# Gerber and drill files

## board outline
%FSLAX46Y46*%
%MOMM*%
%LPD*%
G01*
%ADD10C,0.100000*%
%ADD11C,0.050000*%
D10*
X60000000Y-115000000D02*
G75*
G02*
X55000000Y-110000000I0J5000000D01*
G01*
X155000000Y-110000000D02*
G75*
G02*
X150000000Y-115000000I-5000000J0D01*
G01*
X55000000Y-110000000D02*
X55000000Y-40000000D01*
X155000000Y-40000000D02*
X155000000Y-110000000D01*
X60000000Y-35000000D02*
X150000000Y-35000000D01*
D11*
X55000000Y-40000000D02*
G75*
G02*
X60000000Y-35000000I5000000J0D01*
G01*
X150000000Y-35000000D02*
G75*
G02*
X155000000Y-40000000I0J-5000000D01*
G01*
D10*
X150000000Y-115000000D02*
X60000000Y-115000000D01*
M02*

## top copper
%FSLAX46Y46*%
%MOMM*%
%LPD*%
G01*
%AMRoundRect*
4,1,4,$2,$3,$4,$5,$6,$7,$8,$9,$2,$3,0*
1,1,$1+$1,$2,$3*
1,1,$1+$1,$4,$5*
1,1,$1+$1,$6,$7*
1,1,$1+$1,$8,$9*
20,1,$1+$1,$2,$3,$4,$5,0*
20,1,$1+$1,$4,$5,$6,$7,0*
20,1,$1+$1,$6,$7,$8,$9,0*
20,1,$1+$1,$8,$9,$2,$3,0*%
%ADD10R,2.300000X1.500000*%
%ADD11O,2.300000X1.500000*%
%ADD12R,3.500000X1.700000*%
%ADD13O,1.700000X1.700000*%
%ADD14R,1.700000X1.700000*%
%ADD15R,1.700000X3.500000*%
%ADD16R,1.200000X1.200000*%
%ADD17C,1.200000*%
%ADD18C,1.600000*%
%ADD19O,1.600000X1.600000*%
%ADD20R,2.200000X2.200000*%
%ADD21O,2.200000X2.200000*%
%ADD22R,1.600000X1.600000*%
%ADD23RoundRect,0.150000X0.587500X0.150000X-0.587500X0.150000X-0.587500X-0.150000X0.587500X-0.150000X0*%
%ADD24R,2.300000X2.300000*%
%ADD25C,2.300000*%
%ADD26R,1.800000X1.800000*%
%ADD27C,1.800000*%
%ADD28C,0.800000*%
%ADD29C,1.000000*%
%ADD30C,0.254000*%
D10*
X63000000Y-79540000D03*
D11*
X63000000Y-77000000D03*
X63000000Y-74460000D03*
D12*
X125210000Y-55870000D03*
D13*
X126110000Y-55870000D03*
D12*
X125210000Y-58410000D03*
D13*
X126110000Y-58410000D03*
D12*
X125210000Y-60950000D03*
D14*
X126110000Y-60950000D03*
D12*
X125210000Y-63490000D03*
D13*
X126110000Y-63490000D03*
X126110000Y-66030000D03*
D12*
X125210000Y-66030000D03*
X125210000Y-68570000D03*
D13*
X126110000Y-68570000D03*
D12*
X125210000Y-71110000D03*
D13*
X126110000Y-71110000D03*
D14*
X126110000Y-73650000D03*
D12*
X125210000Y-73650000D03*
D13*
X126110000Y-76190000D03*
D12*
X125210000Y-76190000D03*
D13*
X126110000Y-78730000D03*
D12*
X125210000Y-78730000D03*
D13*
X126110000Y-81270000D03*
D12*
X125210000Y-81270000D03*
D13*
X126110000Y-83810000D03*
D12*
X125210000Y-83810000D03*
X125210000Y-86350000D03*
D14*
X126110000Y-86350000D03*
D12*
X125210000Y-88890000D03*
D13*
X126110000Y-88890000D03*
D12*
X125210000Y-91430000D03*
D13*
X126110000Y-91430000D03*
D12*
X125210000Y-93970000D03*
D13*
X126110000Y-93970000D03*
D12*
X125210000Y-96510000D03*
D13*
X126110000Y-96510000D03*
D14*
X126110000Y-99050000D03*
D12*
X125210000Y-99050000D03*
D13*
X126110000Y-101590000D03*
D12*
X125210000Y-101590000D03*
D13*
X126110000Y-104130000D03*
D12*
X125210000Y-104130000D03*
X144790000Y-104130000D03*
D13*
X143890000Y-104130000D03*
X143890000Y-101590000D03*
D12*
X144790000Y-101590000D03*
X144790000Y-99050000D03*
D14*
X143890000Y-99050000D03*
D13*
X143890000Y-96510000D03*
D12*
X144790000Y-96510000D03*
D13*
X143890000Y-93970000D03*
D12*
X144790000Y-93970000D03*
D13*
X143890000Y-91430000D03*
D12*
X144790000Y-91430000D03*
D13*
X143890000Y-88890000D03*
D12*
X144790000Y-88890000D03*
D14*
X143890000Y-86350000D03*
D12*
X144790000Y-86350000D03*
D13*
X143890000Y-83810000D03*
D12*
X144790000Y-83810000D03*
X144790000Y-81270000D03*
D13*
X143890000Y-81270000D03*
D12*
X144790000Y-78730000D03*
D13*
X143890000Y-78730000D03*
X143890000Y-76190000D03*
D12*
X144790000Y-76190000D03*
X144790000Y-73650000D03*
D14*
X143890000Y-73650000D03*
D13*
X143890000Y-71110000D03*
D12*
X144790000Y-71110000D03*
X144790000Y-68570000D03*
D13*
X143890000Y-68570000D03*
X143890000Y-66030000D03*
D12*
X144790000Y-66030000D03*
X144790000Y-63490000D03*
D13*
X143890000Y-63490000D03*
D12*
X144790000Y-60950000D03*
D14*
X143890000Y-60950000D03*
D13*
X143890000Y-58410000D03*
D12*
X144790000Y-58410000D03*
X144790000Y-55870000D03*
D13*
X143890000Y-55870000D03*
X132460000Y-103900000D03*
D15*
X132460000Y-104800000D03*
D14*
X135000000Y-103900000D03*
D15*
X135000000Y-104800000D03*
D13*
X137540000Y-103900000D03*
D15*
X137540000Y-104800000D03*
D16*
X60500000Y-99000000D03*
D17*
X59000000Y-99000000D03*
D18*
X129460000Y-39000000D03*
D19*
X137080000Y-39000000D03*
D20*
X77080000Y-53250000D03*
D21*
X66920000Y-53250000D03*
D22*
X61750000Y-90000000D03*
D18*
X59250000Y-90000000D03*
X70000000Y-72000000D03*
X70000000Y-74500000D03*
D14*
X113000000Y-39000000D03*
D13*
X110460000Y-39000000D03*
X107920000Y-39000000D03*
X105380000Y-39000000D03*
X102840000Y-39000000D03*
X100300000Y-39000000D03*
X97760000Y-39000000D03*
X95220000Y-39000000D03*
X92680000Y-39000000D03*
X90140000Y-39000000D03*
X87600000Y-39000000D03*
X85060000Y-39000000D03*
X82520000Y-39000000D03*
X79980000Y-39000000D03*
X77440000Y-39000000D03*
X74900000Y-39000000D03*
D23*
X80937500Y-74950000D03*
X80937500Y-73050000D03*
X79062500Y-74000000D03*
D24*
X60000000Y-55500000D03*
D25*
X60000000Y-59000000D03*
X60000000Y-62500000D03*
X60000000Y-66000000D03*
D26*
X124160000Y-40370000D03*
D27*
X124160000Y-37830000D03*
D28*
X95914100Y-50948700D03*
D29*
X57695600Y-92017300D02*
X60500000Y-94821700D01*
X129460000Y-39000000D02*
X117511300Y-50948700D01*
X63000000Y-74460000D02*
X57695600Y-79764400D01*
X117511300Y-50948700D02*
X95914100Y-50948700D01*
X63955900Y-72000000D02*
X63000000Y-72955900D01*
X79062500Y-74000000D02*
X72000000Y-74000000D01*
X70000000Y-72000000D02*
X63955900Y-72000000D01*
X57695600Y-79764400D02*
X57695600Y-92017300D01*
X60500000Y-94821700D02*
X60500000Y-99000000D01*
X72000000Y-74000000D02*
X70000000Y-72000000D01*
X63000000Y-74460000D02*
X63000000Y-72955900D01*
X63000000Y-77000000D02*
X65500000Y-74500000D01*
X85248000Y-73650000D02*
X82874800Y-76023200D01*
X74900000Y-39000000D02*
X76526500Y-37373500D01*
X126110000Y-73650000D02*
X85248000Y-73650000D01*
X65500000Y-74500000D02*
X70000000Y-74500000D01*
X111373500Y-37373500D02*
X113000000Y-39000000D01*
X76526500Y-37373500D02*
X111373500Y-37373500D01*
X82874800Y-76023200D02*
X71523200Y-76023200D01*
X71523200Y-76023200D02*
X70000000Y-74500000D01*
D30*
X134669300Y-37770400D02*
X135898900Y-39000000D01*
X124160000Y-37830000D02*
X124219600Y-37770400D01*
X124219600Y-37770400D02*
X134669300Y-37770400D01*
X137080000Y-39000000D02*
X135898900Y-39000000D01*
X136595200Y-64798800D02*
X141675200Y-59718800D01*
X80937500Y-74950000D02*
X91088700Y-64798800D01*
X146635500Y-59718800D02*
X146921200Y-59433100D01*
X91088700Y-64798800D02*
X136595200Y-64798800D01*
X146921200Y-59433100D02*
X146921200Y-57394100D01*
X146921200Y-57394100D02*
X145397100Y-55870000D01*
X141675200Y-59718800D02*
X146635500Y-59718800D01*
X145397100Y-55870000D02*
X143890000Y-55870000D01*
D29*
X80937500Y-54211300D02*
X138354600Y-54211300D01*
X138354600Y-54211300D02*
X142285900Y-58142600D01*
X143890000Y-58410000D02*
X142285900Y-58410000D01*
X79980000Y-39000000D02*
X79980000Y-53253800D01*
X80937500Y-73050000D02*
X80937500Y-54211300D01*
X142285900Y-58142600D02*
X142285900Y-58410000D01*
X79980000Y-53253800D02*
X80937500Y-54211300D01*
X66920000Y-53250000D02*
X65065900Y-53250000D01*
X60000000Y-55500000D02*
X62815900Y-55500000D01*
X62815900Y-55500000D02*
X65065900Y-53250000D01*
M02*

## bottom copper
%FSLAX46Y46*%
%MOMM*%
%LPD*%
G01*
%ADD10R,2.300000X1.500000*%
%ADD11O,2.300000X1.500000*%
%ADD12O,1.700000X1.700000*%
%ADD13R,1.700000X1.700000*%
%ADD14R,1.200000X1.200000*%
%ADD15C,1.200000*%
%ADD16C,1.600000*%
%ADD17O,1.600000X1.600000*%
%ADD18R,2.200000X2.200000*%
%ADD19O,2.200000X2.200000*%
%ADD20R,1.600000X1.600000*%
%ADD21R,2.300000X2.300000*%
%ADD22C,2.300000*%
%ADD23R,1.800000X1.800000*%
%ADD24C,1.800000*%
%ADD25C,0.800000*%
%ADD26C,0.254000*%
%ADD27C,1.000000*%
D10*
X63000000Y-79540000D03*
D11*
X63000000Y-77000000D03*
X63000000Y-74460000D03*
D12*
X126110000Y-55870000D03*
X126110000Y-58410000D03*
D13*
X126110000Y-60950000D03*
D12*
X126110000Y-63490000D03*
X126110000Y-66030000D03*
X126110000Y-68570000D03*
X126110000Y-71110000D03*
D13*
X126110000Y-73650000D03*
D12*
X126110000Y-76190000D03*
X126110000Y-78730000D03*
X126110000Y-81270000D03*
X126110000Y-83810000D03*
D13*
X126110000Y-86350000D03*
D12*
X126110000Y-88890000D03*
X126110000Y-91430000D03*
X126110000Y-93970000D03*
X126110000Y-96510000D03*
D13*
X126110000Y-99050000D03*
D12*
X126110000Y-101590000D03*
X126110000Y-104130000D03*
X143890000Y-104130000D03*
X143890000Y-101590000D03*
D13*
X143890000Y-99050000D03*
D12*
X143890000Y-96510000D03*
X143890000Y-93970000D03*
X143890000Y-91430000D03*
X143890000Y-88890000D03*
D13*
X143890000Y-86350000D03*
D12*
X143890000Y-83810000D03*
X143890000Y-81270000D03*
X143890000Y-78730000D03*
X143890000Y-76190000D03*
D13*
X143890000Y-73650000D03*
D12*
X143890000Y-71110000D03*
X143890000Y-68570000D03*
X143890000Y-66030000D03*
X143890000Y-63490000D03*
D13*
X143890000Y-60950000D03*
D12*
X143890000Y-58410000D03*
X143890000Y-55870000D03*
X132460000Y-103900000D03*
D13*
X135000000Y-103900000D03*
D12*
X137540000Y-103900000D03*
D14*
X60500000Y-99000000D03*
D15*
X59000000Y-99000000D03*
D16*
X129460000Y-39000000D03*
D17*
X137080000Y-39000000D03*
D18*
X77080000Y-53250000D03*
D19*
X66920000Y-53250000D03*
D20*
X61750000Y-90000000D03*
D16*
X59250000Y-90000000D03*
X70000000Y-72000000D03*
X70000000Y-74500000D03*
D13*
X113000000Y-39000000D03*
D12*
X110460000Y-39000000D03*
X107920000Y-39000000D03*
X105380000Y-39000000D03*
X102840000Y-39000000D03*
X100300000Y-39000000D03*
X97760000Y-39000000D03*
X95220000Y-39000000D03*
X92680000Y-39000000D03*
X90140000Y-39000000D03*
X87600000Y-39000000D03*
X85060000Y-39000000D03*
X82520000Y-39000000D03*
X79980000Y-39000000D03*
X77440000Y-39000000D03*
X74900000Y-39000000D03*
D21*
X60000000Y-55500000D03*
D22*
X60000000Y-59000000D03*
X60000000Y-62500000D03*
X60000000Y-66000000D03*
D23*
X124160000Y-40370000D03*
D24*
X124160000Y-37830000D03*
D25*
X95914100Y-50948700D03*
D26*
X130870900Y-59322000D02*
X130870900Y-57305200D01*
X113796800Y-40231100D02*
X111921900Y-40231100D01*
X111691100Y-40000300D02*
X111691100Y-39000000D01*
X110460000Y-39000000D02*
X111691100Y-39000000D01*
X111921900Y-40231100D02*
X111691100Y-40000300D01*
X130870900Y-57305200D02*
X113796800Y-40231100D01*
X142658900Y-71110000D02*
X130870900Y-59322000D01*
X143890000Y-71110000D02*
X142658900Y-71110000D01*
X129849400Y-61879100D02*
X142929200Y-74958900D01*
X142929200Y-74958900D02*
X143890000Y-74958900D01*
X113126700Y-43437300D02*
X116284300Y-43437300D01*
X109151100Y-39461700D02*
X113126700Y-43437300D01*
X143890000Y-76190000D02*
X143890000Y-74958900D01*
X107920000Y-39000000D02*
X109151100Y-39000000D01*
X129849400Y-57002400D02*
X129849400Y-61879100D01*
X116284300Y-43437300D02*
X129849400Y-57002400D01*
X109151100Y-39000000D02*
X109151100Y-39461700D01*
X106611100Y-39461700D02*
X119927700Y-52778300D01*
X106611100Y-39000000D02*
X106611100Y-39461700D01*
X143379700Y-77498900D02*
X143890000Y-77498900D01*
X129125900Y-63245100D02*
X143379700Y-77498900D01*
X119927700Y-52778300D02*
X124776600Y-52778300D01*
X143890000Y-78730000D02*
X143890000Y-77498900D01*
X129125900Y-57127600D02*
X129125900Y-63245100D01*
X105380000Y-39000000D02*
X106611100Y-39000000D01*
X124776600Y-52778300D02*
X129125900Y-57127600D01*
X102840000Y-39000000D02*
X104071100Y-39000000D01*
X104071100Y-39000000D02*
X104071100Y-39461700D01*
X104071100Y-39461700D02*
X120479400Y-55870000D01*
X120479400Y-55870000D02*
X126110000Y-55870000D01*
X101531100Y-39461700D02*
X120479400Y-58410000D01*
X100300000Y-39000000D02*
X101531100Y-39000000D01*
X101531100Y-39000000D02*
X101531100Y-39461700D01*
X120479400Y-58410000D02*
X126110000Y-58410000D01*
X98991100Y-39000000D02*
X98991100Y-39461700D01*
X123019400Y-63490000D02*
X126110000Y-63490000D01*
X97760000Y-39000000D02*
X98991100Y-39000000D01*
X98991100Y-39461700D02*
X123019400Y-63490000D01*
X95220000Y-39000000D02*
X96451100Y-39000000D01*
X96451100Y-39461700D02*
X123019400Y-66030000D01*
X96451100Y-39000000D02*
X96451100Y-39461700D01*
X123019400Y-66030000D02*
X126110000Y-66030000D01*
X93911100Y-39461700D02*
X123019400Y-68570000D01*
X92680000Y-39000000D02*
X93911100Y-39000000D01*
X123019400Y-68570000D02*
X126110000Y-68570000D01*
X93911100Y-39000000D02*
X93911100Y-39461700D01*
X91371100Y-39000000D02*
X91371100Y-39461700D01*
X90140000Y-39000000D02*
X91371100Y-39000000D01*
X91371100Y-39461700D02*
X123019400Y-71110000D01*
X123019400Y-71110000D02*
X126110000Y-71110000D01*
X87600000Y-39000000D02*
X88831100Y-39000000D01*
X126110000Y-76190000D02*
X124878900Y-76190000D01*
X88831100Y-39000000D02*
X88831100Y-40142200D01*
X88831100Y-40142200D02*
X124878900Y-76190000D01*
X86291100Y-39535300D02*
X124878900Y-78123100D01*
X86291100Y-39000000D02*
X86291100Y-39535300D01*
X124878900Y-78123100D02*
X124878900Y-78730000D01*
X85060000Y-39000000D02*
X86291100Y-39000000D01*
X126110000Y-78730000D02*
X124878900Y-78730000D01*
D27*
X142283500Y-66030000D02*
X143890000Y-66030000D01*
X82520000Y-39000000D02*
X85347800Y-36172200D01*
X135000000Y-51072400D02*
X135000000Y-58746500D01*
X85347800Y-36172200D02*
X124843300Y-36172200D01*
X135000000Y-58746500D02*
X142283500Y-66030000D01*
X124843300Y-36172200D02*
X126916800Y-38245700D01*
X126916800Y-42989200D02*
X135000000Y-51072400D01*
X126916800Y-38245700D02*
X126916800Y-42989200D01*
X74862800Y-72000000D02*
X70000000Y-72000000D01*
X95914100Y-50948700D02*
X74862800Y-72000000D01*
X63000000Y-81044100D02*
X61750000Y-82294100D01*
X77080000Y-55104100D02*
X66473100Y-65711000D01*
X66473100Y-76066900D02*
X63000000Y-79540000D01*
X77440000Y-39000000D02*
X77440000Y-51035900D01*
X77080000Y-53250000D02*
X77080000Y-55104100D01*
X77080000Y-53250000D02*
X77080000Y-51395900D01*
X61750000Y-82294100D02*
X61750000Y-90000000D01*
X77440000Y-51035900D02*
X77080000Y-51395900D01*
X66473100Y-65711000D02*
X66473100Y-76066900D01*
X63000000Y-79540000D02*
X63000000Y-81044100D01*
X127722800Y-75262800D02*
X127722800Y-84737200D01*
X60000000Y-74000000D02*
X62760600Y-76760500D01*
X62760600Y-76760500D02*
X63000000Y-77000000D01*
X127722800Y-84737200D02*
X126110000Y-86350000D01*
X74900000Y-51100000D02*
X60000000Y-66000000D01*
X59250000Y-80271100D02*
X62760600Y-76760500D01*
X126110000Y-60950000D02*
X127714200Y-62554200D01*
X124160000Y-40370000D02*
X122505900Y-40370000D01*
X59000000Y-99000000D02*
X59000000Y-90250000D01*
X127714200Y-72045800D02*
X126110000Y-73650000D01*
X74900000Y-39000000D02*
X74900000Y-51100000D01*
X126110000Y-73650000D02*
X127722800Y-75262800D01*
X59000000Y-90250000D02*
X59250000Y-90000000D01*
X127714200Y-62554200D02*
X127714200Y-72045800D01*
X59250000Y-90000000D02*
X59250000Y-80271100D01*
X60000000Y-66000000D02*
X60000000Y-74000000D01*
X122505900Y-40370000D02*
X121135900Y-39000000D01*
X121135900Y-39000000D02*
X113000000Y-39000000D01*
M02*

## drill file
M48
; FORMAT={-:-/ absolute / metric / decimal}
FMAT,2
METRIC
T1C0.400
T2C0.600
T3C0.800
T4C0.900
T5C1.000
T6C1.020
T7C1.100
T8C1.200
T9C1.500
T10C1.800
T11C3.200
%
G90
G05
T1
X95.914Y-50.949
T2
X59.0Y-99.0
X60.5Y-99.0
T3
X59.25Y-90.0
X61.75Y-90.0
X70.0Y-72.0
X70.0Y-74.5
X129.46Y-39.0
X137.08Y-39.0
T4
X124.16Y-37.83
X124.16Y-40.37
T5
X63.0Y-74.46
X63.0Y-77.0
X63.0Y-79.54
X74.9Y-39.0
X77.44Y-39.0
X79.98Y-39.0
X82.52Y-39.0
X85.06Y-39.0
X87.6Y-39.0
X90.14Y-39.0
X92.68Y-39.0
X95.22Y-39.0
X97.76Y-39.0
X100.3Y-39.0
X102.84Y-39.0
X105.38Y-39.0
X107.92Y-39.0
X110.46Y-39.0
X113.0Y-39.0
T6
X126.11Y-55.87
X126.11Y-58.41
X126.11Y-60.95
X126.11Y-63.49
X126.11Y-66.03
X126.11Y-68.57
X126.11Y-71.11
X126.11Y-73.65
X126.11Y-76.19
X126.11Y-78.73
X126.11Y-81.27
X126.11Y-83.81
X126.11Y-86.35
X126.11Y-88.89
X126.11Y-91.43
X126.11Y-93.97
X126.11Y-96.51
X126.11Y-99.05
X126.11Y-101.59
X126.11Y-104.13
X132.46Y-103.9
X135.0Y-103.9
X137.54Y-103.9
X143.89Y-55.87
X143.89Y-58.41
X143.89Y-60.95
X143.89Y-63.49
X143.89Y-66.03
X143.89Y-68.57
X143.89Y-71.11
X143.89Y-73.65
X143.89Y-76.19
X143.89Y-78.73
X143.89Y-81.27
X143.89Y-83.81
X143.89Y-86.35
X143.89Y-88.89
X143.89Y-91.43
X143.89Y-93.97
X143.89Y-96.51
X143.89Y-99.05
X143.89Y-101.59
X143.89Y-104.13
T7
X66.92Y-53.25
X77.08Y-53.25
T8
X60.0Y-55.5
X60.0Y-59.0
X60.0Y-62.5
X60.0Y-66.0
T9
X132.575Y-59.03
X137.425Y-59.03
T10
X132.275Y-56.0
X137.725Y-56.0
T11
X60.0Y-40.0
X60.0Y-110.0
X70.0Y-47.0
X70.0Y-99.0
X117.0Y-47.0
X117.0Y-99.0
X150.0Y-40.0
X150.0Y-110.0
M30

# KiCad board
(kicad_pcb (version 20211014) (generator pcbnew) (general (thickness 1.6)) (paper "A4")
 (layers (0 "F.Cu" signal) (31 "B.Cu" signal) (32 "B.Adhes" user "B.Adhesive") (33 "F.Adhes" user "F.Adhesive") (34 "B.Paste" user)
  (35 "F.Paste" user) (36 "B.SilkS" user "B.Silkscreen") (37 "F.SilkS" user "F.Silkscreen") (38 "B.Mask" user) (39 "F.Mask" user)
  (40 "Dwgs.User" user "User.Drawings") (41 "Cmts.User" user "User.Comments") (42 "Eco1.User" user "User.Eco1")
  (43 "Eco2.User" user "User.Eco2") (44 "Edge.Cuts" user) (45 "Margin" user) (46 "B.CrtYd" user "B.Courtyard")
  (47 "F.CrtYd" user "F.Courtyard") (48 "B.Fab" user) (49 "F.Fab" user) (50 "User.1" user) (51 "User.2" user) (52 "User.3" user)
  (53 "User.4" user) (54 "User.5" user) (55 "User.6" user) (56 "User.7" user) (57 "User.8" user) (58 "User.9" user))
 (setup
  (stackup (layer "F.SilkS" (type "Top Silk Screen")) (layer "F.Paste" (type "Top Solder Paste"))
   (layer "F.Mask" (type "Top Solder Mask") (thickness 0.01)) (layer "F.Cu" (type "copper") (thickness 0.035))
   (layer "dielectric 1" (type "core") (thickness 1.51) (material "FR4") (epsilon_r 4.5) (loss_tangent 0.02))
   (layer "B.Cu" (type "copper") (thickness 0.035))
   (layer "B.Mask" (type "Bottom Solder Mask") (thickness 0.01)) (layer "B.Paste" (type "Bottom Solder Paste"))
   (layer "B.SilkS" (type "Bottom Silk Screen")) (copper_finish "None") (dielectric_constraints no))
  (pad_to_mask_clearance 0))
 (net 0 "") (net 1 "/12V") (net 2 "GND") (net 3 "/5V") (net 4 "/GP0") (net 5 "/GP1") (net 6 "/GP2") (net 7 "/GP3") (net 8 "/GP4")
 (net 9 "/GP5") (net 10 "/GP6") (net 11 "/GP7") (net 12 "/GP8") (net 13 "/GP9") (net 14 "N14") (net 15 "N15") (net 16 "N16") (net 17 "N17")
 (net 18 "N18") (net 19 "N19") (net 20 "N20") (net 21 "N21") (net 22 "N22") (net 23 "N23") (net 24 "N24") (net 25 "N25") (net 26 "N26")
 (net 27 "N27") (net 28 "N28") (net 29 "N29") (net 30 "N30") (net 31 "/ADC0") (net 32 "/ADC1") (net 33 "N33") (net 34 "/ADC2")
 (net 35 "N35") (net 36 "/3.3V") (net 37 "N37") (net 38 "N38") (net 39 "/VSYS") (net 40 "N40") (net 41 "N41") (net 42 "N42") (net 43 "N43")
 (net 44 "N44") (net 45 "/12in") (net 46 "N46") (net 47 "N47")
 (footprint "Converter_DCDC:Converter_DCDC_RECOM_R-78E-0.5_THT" (layer "F.Cu") (at 63 79.54 90)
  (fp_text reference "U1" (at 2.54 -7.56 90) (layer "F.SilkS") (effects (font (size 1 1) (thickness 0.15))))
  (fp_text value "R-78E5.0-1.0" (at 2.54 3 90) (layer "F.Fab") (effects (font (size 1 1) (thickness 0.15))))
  (pad "1" thru_hole rect (at 0 0 90) (size 1.5 2.3) (drill 1) (layers *.Cu *.Mask) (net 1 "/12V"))
  (pad "2" thru_hole oval (at 2.54 0 90) (size 1.5 2.3) (drill 1) (layers *.Cu *.Mask) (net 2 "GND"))
  (pad "3" thru_hole oval (at 5.08 0 90) (size 1.5 2.3) (drill 1) (layers *.Cu *.Mask) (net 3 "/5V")))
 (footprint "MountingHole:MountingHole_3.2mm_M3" (layer "F.Cu") (at 117 99)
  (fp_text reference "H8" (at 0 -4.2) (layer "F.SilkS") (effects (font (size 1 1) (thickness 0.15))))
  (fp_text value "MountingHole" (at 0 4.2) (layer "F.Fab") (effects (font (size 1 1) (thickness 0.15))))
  (pad "" np_thru_hole circle (at 0 0) (size 3.2 3.2) (drill 3.2) (layers *.Cu *.Mask)))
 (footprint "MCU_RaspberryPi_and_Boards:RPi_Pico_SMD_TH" (layer "F.Cu") (at 135 80)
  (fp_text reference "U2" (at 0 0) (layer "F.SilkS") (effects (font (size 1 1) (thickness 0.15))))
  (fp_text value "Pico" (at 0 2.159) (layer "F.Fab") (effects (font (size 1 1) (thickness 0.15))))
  (pad "" np_thru_hole oval (at -2.725 -24) (size 1.8 1.8) (drill 1.8) (layers *.Cu *.Mask))
  (pad "" np_thru_hole oval (at -2.425 -20.97) (size 1.5 1.5) (drill 1.5) (layers *.Cu *.Mask))
  (pad "" np_thru_hole oval (at 2.425 -20.97) (size 1.5 1.5) (drill 1.5) (layers *.Cu *.Mask))
  (pad "" np_thru_hole oval (at 2.725 -24) (size 1.8 1.8) (drill 1.8) (layers *.Cu *.Mask))
  (pad "1" smd rect (at -8.89 -24.13) (size 3.5 1.7) (drill (offset -0.9 0)) (layers "F.Cu" "F.Mask") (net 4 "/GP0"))
  (pad "1" thru_hole oval (at -8.89 -24.13) (size 1.7 1.7) (drill 1.02) (layers *.Cu *.Mask) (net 4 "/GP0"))
  (pad "2" smd rect (at -8.89 -21.59) (size 3.5 1.7) (drill (offset -0.9 0)) (layers "F.Cu" "F.Mask") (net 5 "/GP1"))
  (pad "2" thru_hole oval (at -8.89 -21.59) (size 1.7 1.7) (drill 1.02) (layers *.Cu *.Mask) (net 5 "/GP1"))
  (pad "3" smd rect (at -8.89 -19.05) (size 3.5 1.7) (drill (offset -0.9 0)) (layers "F.Cu" "F.Mask") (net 2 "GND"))
  (pad "3" thru_hole rect (at -8.89 -19.05) (size 1.7 1.7) (drill 1.02) (layers *.Cu *.Mask) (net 2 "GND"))
  (pad "4" smd rect (at -8.89 -16.51) (size 3.5 1.7) (drill (offset -0.9 0)) (layers "F.Cu" "F.Mask") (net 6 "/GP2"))
  (pad "4" thru_hole oval (at -8.89 -16.51) (size 1.7 1.7) (drill 1.02) (layers *.Cu *.Mask) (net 6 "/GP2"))
  (pad "5" thru_hole oval (at -8.89 -13.97) (size 1.7 1.7) (drill 1.02) (layers *.Cu *.Mask) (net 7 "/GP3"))
  (pad "5" smd rect (at -8.89 -13.97) (size 3.5 1.7) (drill (offset -0.9 0)) (layers "F.Cu" "F.Mask") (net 7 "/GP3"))
  (pad "6" smd rect (at -8.89 -11.43) (size 3.5 1.7) (drill (offset -0.9 0)) (layers "F.Cu" "F.Mask") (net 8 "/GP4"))
  (pad "6" thru_hole oval (at -8.89 -11.43) (size 1.7 1.7) (drill 1.02) (layers *.Cu *.Mask) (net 8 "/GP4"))
  (pad "7" smd rect (at -8.89 -8.89) (size 3.5 1.7) (drill (offset -0.9 0)) (layers "F.Cu" "F.Mask") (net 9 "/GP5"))
  (pad "7" thru_hole oval (at -8.89 -8.89) (size 1.7 1.7) (drill 1.02) (layers *.Cu *.Mask) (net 9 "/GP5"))
  (pad "8" thru_hole rect (at -8.89 -6.35) (size 1.7 1.7) (drill 1.02) (layers *.Cu *.Mask) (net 2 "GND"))
  (pad "8" smd rect (at -8.89 -6.35) (size 3.5 1.7) (drill (offset -0.9 0)) (layers "F.Cu" "F.Mask") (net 2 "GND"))
  (pad "9" thru_hole oval (at -8.89 -3.81) (size 1.7 1.7) (drill 1.02) (layers *.Cu *.Mask) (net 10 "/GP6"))
  (pad "9" smd rect (at -8.89 -3.81) (size 3.5 1.7) (drill (offset -0.9 0)) (layers "F.Cu" "F.Mask") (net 10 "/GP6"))
  (pad "10" thru_hole oval (at -8.89 -1.27) (size 1.7 1.7) (drill 1.02) (layers *.Cu *.Mask) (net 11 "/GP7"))
  (pad "10" smd rect (at -8.89 -1.27) (size 3.5 1.7) (drill (offset -0.9 0)) (layers "F.Cu" "F.Mask") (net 11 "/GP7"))
  (pad "11" thru_hole oval (at -8.89 1.27) (size 1.7 1.7) (drill 1.02) (layers *.Cu *.Mask) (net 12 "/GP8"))
  (pad "11" smd rect (at -8.89 1.27) (size 3.5 1.7) (drill (offset -0.9 0)) (layers "F.Cu" "F.Mask") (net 12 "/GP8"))
  (pad "12" thru_hole oval (at -8.89 3.81) (size 1.7 1.7) (drill 1.02) (layers *.Cu *.Mask) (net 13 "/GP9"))
  (pad "12" smd rect (at -8.89 3.81) (size 3.5 1.7) (drill (offset -0.9 0)) (layers "F.Cu" "F.Mask") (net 13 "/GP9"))
  (pad "13" smd rect (at -8.89 6.35) (size 3.5 1.7) (drill (offset -0.9 0)) (layers "F.Cu" "F.Mask") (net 2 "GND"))
  (pad "13" thru_hole rect (at -8.89 6.35) (size 1.7 1.7) (drill 1.02) (layers *.Cu *.Mask) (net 2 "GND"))
  (pad "14" smd rect (at -8.89 8.89) (size 3.5 1.7) (drill (offset -0.9 0)) (layers "F.Cu" "F.Mask") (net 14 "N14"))
  (pad "14" thru_hole oval (at -8.89 8.89) (size 1.7 1.7) (drill 1.02) (layers *.Cu *.Mask) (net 14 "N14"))
  (pad "15" smd rect (at -8.89 11.43) (size 3.5 1.7) (drill (offset -0.9 0)) (layers "F.Cu" "F.Mask") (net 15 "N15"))
  (pad "15" thru_hole oval (at -8.89 11.43) (size 1.7 1.7) (drill 1.02) (layers *.Cu *.Mask) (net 15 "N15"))
  (pad "16" smd rect (at -8.89 13.97) (size 3.5 1.7) (drill (offset -0.9 0)) (layers "F.Cu" "F.Mask") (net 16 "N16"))
  (pad "16" thru_hole oval (at -8.89 13.97) (size 1.7 1.7) (drill 1.02) (layers *.Cu *.Mask) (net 16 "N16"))
  (pad "17" smd rect (at -8.89 16.51) (size 3.5 1.7) (drill (offset -0.9 0)) (layers "F.Cu" "F.Mask") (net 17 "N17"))
  (pad "17" thru_hole oval (at -8.89 16.51) (size 1.7 1.7) (drill 1.02) (layers *.Cu *.Mask) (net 17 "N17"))
  (pad "18" thru_hole rect (at -8.89 19.05) (size 1.7 1.7) (drill 1.02) (layers *.Cu *.Mask) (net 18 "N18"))
  (pad "18" smd rect (at -8.89 19.05) (size 3.5 1.7) (drill (offset -0.9 0)) (layers "F.Cu" "F.Mask") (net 18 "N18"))
  (pad "19" thru_hole oval (at -8.89 21.59) (size 1.7 1.7) (drill 1.02) (layers *.Cu *.Mask) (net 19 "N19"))
  (pad "19" smd rect (at -8.89 21.59) (size 3.5 1.7) (drill (offset -0.9 0)) (layers "F.Cu" "F.Mask") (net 19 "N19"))
  (pad "20" thru_hole oval (at -8.89 24.13) (size 1.7 1.7) (drill 1.02) (layers *.Cu *.Mask) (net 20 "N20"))
  (pad "20" smd rect (at -8.89 24.13) (size 3.5 1.7) (drill (offset -0.9 0)) (layers "F.Cu" "F.Mask") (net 20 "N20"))
  (pad "21" smd rect (at 8.89 24.13) (size 3.5 1.7) (drill (offset 0.9 0)) (layers "F.Cu" "F.Mask") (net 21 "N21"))
  (pad "21" thru_hole oval (at 8.89 24.13) (size 1.7 1.7) (drill 1.02) (layers *.Cu *.Mask) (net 21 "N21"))
  (pad "22" thru_hole oval (at 8.89 21.59) (size 1.7 1.7) (drill 1.02) (layers *.Cu *.Mask) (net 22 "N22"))
  (pad "22" smd rect (at 8.89 21.59) (size 3.5 1.7) (drill (offset 0.9 0)) (layers "F.Cu" "F.Mask") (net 22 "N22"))
  (pad "23" smd rect (at 8.89 19.05) (size 3.5 1.7) (drill (offset 0.9 0)) (layers "F.Cu" "F.Mask") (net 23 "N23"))
  (pad "23" thru_hole rect (at 8.89 19.05) (size 1.7 1.7) (drill 1.02) (layers *.Cu *.Mask) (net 23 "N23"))
  (pad "24" thru_hole oval (at 8.89 16.51) (size 1.7 1.7) (drill 1.02) (layers *.Cu *.Mask) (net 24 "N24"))
  (pad "24" smd rect (at 8.89 16.51) (size 3.5 1.7) (drill (offset 0.9 0)) (layers "F.Cu" "F.Mask") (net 24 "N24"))
  (pad "25" thru_hole oval (at 8.89 13.97) (size 1.7 1.7) (drill 1.02) (layers *.Cu *.Mask) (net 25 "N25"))
  (pad "25" smd rect (at 8.89 13.97) (size 3.5 1.7) (drill (offset 0.9 0)) (layers "F.Cu" "F.Mask") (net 25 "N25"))
  (pad "26" thru_hole oval (at 8.89 11.43) (size 1.7 1.7) (drill 1.02) (layers *.Cu *.Mask) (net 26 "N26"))
  (pad "26" smd rect (at 8.89 11.43) (size 3.5 1.7) (drill (offset 0.9 0)) (layers "F.Cu" "F.Mask") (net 26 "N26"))
  (pad "27" thru_hole oval (at 8.89 8.89) (size 1.7 1.7) (drill 1.02) (layers *.Cu *.Mask) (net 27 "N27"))
  (pad "27" smd rect (at 8.89 8.89) (size 3.5 1.7) (drill (offset 0.9 0)) (layers "F.Cu" "F.Mask") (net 27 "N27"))
  (pad "28" thru_hole rect (at 8.89 6.35) (size 1.7 1.7) (drill 1.02) (layers *.Cu *.Mask) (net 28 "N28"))
  (pad "28" smd rect (at 8.89 6.35) (size 3.5 1.7) (drill (offset 0.9 0)) (layers "F.Cu" "F.Mask") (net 28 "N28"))
  (pad "29" thru_hole oval (at 8.89 3.81) (size 1.7 1.7) (drill 1.02) (layers *.Cu *.Mask) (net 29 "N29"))
  (pad "29" smd rect (at 8.89 3.81) (size 3.5 1.7) (drill (offset 0.9 0)) (layers "F.Cu" "F.Mask") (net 29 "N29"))
  (pad "30" smd rect (at 8.89 1.27) (size 3.5 1.7) (drill (offset 0.9 0)) (layers "F.Cu" "F.Mask") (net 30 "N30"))
  (pad "30" thru_hole oval (at 8.89 1.27) (size 1.7 1.7) (drill 1.02) (layers *.Cu *.Mask) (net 30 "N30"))
  (pad "31" smd rect (at 8.89 -1.27) (size 3.5 1.7) (drill (offset 0.9 0)) (layers "F.Cu" "F.Mask") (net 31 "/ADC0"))
  (pad "31" thru_hole oval (at 8.89 -1.27) (size 1.7 1.7) (drill 1.02) (layers *.Cu *.Mask) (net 31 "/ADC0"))
  (pad "32" thru_hole oval (at 8.89 -3.81) (size 1.7 1.7) (drill 1.02) (layers *.Cu *.Mask) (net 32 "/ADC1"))
  (pad "32" smd rect (at 8.89 -3.81) (size 3.5 1.7) (drill (offset 0.9 0)) (layers "F.Cu" "F.Mask") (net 32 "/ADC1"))
  (pad "33" smd rect (at 8.89 -6.35) (size 3.5 1.7) (drill (offset 0.9 0)) (layers "F.Cu" "F.Mask") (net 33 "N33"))
  (pad "33" thru_hole rect (at 8.89 -6.35) (size 1.7 1.7) (drill 1.02) (layers *.Cu *.Mask) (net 33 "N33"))
  (pad "34" thru_hole oval (at 8.89 -8.89) (size 1.7 1.7) (drill 1.02) (layers *.Cu *.Mask) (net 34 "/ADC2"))
  (pad "34" smd rect (at 8.89 -8.89) (size 3.5 1.7) (drill (offset 0.9 0)) (layers "F.Cu" "F.Mask") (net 34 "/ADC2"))
  (pad "35" smd rect (at 8.89 -11.43) (size 3.5 1.7) (drill (offset 0.9 0)) (layers "F.Cu" "F.Mask") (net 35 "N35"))
  (pad "35" thru_hole oval (at 8.89 -11.43) (size 1.7 1.7) (drill 1.02) (layers *.Cu *.Mask) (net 35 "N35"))
  (pad "36" thru_hole oval (at 8.89 -13.97) (size 1.7 1.7) (drill 1.02) (layers *.Cu *.Mask) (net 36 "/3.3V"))
  (pad "36" smd rect (at 8.89 -13.97) (size 3.5 1.7) (drill (offset 0.9 0)) (layers "F.Cu" "F.Mask") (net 36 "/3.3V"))
  (pad "37" smd rect (at 8.89 -16.51) (size 3.5 1.7) (drill (offset 0.9 0)) (layers "F.Cu" "F.Mask") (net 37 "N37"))
  (pad "37" thru_hole oval (at 8.89 -16.51) (size 1.7 1.7) (drill 1.02) (layers *.Cu *.Mask) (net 37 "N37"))
  (pad "38" smd rect (at 8.89 -19.05) (size 3.5 1.7) (drill (offset 0.9 0)) (layers "F.Cu" "F.Mask") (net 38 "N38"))
  (pad "38" thru_hole rect (at 8.89 -19.05) (size 1.7 1.7) (drill 1.02) (layers *.Cu *.Mask) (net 38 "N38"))
  (pad "39" thru_hole oval (at 8.89 -21.59) (size 1.7 1.7) (drill 1.02) (layers *.Cu *.Mask) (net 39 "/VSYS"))
  (pad "39" smd rect (at 8.89 -21.59) (size 3.5 1.7) (drill (offset 0.9 0)) (layers "F.Cu" "F.Mask") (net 39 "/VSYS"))
  (pad "40" smd rect (at 8.89 -24.13) (size 3.5 1.7) (drill (offset 0.9 0)) (layers "F.Cu" "F.Mask") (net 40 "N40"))
  (pad "40" thru_hole oval (at 8.89 -24.13) (size 1.7 1.7) (drill 1.02) (layers *.Cu *.Mask) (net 40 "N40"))
  (pad "41" thru_hole oval (at -2.54 23.9) (size 1.7 1.7) (drill 1.02) (layers *.Cu *.Mask) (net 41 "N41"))
  (pad "41" smd rect (at -2.54 23.9 90) (size 3.5 1.7) (drill (offset -0.9 0)) (layers "F.Cu" "F.Mask") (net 41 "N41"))
  (pad "42" thru_hole rect (at 0 23.9) (size 1.7 1.7) (drill 1.02) (layers *.Cu *.Mask) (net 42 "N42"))
  (pad "42" smd rect (at 0 23.9 90) (size 3.5 1.7) (drill (offset -0.9 0)) (layers "F.Cu" "F.Mask") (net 42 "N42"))
  (pad "43" thru_hole oval (at 2.54 23.9) (size 1.7 1.7) (drill 1.02) (layers *.Cu *.Mask) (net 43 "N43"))
  (pad "43" smd rect (at 2.54 23.9 90) (size 3.5 1.7) (drill (offset -0.9 0)) (layers "F.Cu" "F.Mask") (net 43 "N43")))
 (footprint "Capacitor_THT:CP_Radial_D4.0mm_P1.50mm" (layer "F.Cu") (at 60.5 99 180)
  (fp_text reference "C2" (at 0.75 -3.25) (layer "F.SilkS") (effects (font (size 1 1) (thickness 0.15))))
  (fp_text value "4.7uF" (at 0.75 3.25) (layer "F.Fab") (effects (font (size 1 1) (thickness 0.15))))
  (pad "1" thru_hole rect (at 0 0 180) (size 1.2 1.2) (drill 0.6) (layers *.Cu *.Mask) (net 3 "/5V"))
  (pad "2" thru_hole circle (at 1.5 0 180) (size 1.2 1.2) (drill 0.6) (layers *.Cu *.Mask) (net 2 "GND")))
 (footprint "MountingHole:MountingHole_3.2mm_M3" (layer "F.Cu") (at 70 99)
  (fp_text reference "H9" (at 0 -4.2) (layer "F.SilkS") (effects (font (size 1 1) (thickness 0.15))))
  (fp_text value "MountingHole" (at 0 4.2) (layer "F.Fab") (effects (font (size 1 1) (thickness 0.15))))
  (pad "" np_thru_hole circle (at 0 0) (size 3.2 3.2) (drill 3.2) (layers *.Cu *.Mask)))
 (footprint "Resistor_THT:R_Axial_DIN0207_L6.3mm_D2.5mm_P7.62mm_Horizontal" (layer "F.Cu") (at 129.46 39)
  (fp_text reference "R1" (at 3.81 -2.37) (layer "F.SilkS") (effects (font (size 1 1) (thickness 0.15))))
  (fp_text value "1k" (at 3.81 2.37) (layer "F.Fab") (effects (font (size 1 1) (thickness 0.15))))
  (pad "1" thru_hole circle (at 0 0) (size 1.6 1.6) (drill 0.8) (layers *.Cu *.Mask) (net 3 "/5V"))
  (pad "2" thru_hole oval (at 7.62 0) (size 1.6 1.6) (drill 0.8) (layers *.Cu *.Mask) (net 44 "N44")))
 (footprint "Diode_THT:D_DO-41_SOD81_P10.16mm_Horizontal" (layer "F.Cu") (at 77.08 53.25 180)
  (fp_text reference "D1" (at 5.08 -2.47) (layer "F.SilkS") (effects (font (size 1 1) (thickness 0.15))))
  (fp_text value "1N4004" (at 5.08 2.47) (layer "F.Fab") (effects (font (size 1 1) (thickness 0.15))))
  (pad "1" thru_hole rect (at 0 0 180) (size 2.2 2.2) (drill 1.1) (layers *.Cu *.Mask) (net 1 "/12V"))
  (pad "2" thru_hole oval (at 10.16 0 180) (size 2.2 2.2) (drill 1.1) (layers *.Cu *.Mask) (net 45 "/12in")))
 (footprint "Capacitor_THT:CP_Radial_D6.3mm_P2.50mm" (layer "F.Cu") (at 61.75 90 180)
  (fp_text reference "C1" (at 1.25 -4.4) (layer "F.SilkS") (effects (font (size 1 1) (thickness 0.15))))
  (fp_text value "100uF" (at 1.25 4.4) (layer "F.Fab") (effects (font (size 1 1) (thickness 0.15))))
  (pad "1" thru_hole rect (at 0 0 180) (size 1.6 1.6) (drill 0.8) (layers *.Cu *.Mask) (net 1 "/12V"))
  (pad "2" thru_hole circle (at 2.5 0 180) (size 1.6 1.6) (drill 0.8) (layers *.Cu *.Mask) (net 2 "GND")))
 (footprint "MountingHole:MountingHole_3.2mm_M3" (layer "F.Cu") (at 117 47)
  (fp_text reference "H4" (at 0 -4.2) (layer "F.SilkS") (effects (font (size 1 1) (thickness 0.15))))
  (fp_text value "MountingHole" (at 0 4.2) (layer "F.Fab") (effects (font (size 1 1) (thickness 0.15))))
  (pad "" np_thru_hole circle (at 0 0) (size 3.2 3.2) (drill 3.2) (layers *.Cu *.Mask)))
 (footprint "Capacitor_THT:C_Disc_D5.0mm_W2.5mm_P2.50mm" (layer "F.Cu") (at 70 72 -90)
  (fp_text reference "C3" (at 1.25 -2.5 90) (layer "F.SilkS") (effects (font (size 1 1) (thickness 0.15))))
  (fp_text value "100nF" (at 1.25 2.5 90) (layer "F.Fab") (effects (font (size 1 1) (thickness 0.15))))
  (pad "1" thru_hole circle (at 0 0 270) (size 1.6 1.6) (drill 0.8) (layers *.Cu *.Mask) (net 3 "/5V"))
  (pad "2" thru_hole circle (at 2.5 0 270) (size 1.6 1.6) (drill 0.8) (layers *.Cu *.Mask) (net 2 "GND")))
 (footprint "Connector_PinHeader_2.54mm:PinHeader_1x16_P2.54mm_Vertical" (layer "F.Cu") (at 113 39 -90)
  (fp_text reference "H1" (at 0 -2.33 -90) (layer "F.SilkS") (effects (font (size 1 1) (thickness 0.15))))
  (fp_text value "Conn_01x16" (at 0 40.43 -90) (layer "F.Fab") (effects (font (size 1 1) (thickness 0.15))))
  (pad "1" thru_hole rect (at 0 0 270) (size 1.7 1.7) (drill 1) (layers *.Cu *.Mask) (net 2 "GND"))
  (pad "2" thru_hole oval (at 0 2.54 270) (size 1.7 1.7) (drill 1) (layers *.Cu *.Mask) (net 34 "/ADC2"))
  (pad "3" thru_hole oval (at 0 5.08 270) (size 1.7 1.7) (drill 1) (layers *.Cu *.Mask) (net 32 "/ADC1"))
  (pad "4" thru_hole oval (at 0 7.62 270) (size 1.7 1.7) (drill 1) (layers *.Cu *.Mask) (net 31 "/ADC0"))
  (pad "5" thru_hole oval (at 0 10.16 270) (size 1.7 1.7) (drill 1) (layers *.Cu *.Mask) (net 4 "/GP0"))
  (pad "6" thru_hole oval (at 0 12.7 270) (size 1.7 1.7) (drill 1) (layers *.Cu *.Mask) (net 5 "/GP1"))
  (pad "7" thru_hole oval (at 0 15.24 270) (size 1.7 1.7) (drill 1) (layers *.Cu *.Mask) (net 6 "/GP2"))
  (pad "8" thru_hole oval (at 0 17.78 270) (size 1.7 1.7) (drill 1) (layers *.Cu *.Mask) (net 7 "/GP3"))
  (pad "9" thru_hole oval (at 0 20.32 270) (size 1.7 1.7) (drill 1) (layers *.Cu *.Mask) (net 8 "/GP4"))
  (pad "10" thru_hole oval (at 0 22.86 270) (size 1.7 1.7) (drill 1) (layers *.Cu *.Mask) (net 9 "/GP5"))
  (pad "11" thru_hole oval (at 0 25.4 270) (size 1.7 1.7) (drill 1) (layers *.Cu *.Mask) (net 10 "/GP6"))
  (pad "12" thru_hole oval (at 0 27.94 270) (size 1.7 1.7) (drill 1) (layers *.Cu *.Mask) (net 11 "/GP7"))
  (pad "13" thru_hole oval (at 0 30.48 270) (size 1.7 1.7) (drill 1) (layers *.Cu *.Mask) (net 36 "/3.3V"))
  (pad "14" thru_hole oval (at 0 33.02 270) (size 1.7 1.7) (drill 1) (layers *.Cu *.Mask) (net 39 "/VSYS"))
  (pad "15" thru_hole oval (at 0 35.56 270) (size 1.7 1.7) (drill 1) (layers *.Cu *.Mask) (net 1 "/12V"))
  (pad "16" thru_hole oval (at 0 38.1 270) (size 1.7 1.7) (drill 1) (layers *.Cu *.Mask) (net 2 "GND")))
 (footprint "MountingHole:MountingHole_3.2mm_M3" (layer "F.Cu") (at 60 40)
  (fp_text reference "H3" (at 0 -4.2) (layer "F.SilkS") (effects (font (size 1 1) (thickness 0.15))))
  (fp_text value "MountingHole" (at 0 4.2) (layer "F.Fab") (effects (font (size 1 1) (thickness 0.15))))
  (pad "" np_thru_hole circle (at 0 0) (size 3.2 3.2) (drill 3.2) (layers *.Cu *.Mask)))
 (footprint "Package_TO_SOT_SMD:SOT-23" (layer "F.Cu") (at 80 74 180)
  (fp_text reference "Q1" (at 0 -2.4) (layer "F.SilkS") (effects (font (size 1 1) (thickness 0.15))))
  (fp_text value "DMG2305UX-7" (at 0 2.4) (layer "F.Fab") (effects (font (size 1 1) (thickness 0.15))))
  (pad "1" smd roundrect (at -0.9375 -0.95 180) (size 1.475 0.6) (layers "F.Cu" "F.Paste" "F.Mask") (roundrect_rratio 0.25) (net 40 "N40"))
  (pad "2" smd roundrect (at -0.9375 0.95 180) (size 1.475 0.6) (layers "F.Cu" "F.Paste" "F.Mask") (roundrect_rratio 0.25) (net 39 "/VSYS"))
  (pad "3" smd roundrect (at 0.9375 0 180) (size 1.475 0.6) (layers "F.Cu" "F.Paste" "F.Mask") (roundrect_rratio 0.25) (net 3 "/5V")))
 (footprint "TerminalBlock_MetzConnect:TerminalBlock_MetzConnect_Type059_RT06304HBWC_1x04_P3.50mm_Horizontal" (layer "F.Cu")
  (at 60 55.5 -90)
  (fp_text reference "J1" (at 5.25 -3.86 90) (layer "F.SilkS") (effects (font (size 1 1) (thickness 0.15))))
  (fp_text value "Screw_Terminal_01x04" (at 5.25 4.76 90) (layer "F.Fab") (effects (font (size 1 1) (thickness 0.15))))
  (pad "1" thru_hole rect (at 0 0 270) (size 2.3 2.3) (drill 1.2) (layers *.Cu *.Mask) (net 45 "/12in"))
  (pad "2" thru_hole circle (at 3.5 0 270) (size 2.3 2.3) (drill 1.2) (layers *.Cu *.Mask) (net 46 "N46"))
  (pad "3" thru_hole circle (at 7 0 270) (size 2.3 2.3) (drill 1.2) (layers *.Cu *.Mask) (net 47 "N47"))
  (pad "4" thru_hole circle (at 10.5 0 270) (size 2.3 2.3) (drill 1.2) (layers *.Cu *.Mask) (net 2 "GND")))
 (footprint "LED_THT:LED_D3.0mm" (layer "F.Cu") (at 124.16 40.37 90)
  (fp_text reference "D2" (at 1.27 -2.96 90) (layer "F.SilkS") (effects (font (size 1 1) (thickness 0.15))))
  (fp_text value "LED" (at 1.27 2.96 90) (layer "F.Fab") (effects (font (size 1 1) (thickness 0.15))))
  (pad "1" thru_hole rect (at 0 0 90) (size 1.8 1.8) (drill 0.9) (layers *.Cu *.Mask) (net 2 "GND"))
  (pad "2" thru_hole circle (at 2.54 0 90) (size 1.8 1.8) (drill 0.9) (layers *.Cu *.Mask) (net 44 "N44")))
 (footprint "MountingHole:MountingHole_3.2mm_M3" (layer "F.Cu") (at 70 47)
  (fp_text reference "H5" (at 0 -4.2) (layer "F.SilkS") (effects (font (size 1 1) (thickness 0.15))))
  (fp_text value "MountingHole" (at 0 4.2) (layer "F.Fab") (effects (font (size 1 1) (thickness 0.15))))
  (pad "" np_thru_hole circle (at 0 0) (size 3.2 3.2) (drill 3.2) (layers *.Cu *.Mask)))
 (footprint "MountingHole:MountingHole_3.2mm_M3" (layer "F.Cu") (at 150 110)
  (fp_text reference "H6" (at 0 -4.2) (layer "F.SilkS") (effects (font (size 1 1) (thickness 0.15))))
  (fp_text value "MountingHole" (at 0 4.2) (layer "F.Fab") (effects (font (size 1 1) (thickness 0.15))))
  (pad "" np_thru_hole circle (at 0 0) (size 3.2 3.2) (drill 3.2) (layers *.Cu *.Mask)))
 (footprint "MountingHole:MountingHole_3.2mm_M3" (layer "F.Cu") (at 60 110)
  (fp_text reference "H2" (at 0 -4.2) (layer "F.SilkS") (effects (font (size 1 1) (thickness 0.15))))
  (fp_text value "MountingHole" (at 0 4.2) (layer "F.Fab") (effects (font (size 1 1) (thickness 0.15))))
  (pad "" np_thru_hole circle (at 0 0) (size 3.2 3.2) (drill 3.2) (layers *.Cu *.Mask)))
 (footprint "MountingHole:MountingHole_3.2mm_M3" (layer "F.Cu") (at 150 40)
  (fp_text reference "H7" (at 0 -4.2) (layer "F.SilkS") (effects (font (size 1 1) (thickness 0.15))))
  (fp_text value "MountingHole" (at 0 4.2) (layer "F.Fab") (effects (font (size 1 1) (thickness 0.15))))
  (pad "" np_thru_hole circle (at 0 0) (size 3.2 3.2) (drill 3.2) (layers *.Cu *.Mask)))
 (gr_arc (start 60 115) (mid 56.464466 113.535534) (end 55 110) (layer "Edge.Cuts") (width 0.1))
 (gr_arc (start 155 110) (mid 153.535534 113.535534) (end 150 115) (layer "Edge.Cuts") (width 0.1))
 (gr_line (start 55 110) (end 55 40) (layer "Edge.Cuts") (width 0.1))
 (gr_line (start 155 40) (end 155 110) (layer "Edge.Cuts") (width 0.1))
 (gr_line (start 60 35) (end 150 35) (layer "Edge.Cuts") (width 0.1))
 (gr_arc (start 55 40) (mid 56.464466 36.464466) (end 60 35) (layer "Edge.Cuts") (width 0.05))
 (gr_arc (start 150 35) (mid 153.535534 36.464466) (end 155 40) (layer "Edge.Cuts") (width 0.05))
 (gr_line (start 150 115) (end 60 115) (layer "Edge.Cuts") (width 0.1))
 (segment (start 130.8709 59.322) (end 130.8709 57.3052) (width 0.254) (layer "B.Cu") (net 34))
 (segment (start 113.7968 40.2311) (end 111.9219 40.2311) (width 0.254) (layer "B.Cu") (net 34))
 (segment (start 111.6911 40.0003) (end 111.6911 39) (width 0.254) (layer "B.Cu") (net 34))
 (segment (start 110.46 39) (end 111.6911 39) (width 0.254) (layer "B.Cu") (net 34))
 (segment (start 111.9219 40.2311) (end 111.6911 40.0003) (width 0.254) (layer "B.Cu") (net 34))
 (segment (start 130.8709 57.3052) (end 113.7968 40.2311) (width 0.254) (layer "B.Cu") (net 34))
 (segment (start 142.6589 71.11) (end 130.8709 59.322) (width 0.254) (layer "B.Cu") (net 34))
 (segment (start 143.89 71.11) (end 142.6589 71.11) (width 0.254) (layer "B.Cu") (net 34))
 (segment (start 129.8494 61.8791) (end 142.9292 74.9589) (width 0.254) (layer "B.Cu") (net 32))
 (segment (start 142.9292 74.9589) (end 143.89 74.9589) (width 0.254) (layer "B.Cu") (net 32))
 (segment (start 113.1267 43.4373) (end 116.2843 43.4373) (width 0.254) (layer "B.Cu") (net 32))
 (segment (start 109.1511 39.4617) (end 113.1267 43.4373) (width 0.254) (layer "B.Cu") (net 32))
 (segment (start 143.89 76.19) (end 143.89 74.9589) (width 0.254) (layer "B.Cu") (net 32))
 (segment (start 107.92 39) (end 109.1511 39) (width 0.254) (layer "B.Cu") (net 32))
 (segment (start 129.8494 57.0024) (end 129.8494 61.8791) (width 0.254) (layer "B.Cu") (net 32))
 (segment (start 116.2843 43.4373) (end 129.8494 57.0024) (width 0.254) (layer "B.Cu") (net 32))
 (segment (start 109.1511 39) (end 109.1511 39.4617) (width 0.254) (layer "B.Cu") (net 32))
 (segment (start 106.6111 39.4617) (end 119.9277 52.7783) (width 0.254) (layer "B.Cu") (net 31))
 (segment (start 106.6111 39) (end 106.6111 39.4617) (width 0.254) (layer "B.Cu") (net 31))
 (segment (start 143.3797 77.4989) (end 143.89 77.4989) (width 0.254) (layer "B.Cu") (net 31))
 (segment (start 129.1259 63.2451) (end 143.3797 77.4989) (width 0.254) (layer "B.Cu") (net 31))
 (segment (start 119.9277 52.7783) (end 124.7766 52.7783) (width 0.254) (layer "B.Cu") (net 31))
 (segment (start 143.89 78.73) (end 143.89 77.4989) (width 0.254) (layer "B.Cu") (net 31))
 (segment (start 129.1259 57.1276) (end 129.1259 63.2451) (width 0.254) (layer "B.Cu") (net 31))
 (segment (start 105.38 39) (end 106.6111 39) (width 0.254) (layer "B.Cu") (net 31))
 (segment (start 124.7766 52.7783) (end 129.1259 57.1276) (width 0.254) (layer "B.Cu") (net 31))
 (segment (start 102.84 39) (end 104.0711 39) (width 0.254) (layer "B.Cu") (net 4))
 (segment (start 104.0711 39) (end 104.0711 39.4617) (width 0.254) (layer "B.Cu") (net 4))
 (segment (start 104.0711 39.4617) (end 120.4794 55.87) (width 0.254) (layer "B.Cu") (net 4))
 (segment (start 120.4794 55.87) (end 126.11 55.87) (width 0.254) (layer "B.Cu") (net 4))
 (segment (start 101.5311 39.4617) (end 120.4794 58.41) (width 0.254) (layer "B.Cu") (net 5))
 (segment (start 100.3 39) (end 101.5311 39) (width 0.254) (layer "B.Cu") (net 5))
 (segment (start 101.5311 39) (end 101.5311 39.4617) (width 0.254) (layer "B.Cu") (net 5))
 (segment (start 120.4794 58.41) (end 126.11 58.41) (width 0.254) (layer "B.Cu") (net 5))
 (segment (start 98.9911 39) (end 98.9911 39.4617) (width 0.254) (layer "B.Cu") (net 6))
 (segment (start 123.0194 63.49) (end 126.11 63.49) (width 0.254) (layer "B.Cu") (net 6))
 (segment (start 97.76 39) (end 98.9911 39) (width 0.254) (layer "B.Cu") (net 6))
 (segment (start 98.9911 39.4617) (end 123.0194 63.49) (width 0.254) (layer "B.Cu") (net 6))
 (segment (start 95.22 39) (end 96.4511 39) (width 0.254) (layer "B.Cu") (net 7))
 (segment (start 96.4511 39.4617) (end 123.0194 66.03) (width 0.254) (layer "B.Cu") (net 7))
 (segment (start 96.4511 39) (end 96.4511 39.4617) (width 0.254) (layer "B.Cu") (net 7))
 (segment (start 123.0194 66.03) (end 126.11 66.03) (width 0.254) (layer "B.Cu") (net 7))
 (segment (start 93.9111 39.4617) (end 123.0194 68.57) (width 0.254) (layer "B.Cu") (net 8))
 (segment (start 92.68 39) (end 93.9111 39) (width 0.254) (layer "B.Cu") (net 8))
 (segment (start 123.0194 68.57) (end 126.11 68.57) (width 0.254) (layer "B.Cu") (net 8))
 (segment (start 93.9111 39) (end 93.9111 39.4617) (width 0.254) (layer "B.Cu") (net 8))
 (segment (start 91.3711 39) (end 91.3711 39.4617) (width 0.254) (layer "B.Cu") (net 9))
 (segment (start 90.14 39) (end 91.3711 39) (width 0.254) (layer "B.Cu") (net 9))
 (segment (start 91.3711 39.4617) (end 123.0194 71.11) (width 0.254) (layer "B.Cu") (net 9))
 (segment (start 123.0194 71.11) (end 126.11 71.11) (width 0.254) (layer "B.Cu") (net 9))
 (segment (start 87.6 39) (end 88.8311 39) (width 0.254) (layer "B.Cu") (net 10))
 (segment (start 126.11 76.19) (end 124.8789 76.19) (width 0.254) (layer "B.Cu") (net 10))
 (segment (start 88.8311 39) (end 88.8311 40.1422) (width 0.254) (layer "B.Cu") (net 10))
 (segment (start 88.8311 40.1422) (end 124.8789 76.19) (width 0.254) (layer "B.Cu") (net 10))
 (segment (start 86.2911 39.5353) (end 124.8789 78.1231) (width 0.254) (layer "B.Cu") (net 11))
 (segment (start 86.2911 39) (end 86.2911 39.5353) (width 0.254) (layer "B.Cu") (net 11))
 (segment (start 124.8789 78.1231) (end 124.8789 78.73) (width 0.254) (layer "B.Cu") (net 11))
 (segment (start 85.06 39) (end 86.2911 39) (width 0.254) (layer "B.Cu") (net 11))
 (segment (start 126.11 78.73) (end 124.8789 78.73) (width 0.254) (layer "B.Cu") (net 11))
 (segment (start 142.2835 66.03) (end 143.89 66.03) (width 1) (layer "B.Cu") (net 36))
 (segment (start 82.52 39) (end 85.3478 36.1722) (width 1) (layer "B.Cu") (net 36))
 (segment (start 135 51.0724) (end 135 58.7465) (width 1) (layer "B.Cu") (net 36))
 (segment (start 85.3478 36.1722) (end 124.8433 36.1722) (width 1) (layer "B.Cu") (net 36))
 (segment (start 135 58.7465) (end 142.2835 66.03) (width 1) (layer "B.Cu") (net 36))
 (segment (start 124.8433 36.1722) (end 126.9168 38.2457) (width 1) (layer "B.Cu") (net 36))
 (segment (start 126.9168 42.9892) (end 135 51.0724) (width 1) (layer "B.Cu") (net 36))
 (segment (start 126.9168 38.2457) (end 126.9168 42.9892) (width 1) (layer "B.Cu") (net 36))
 (segment (start 57.6956 92.0173) (end 60.5 94.8217) (width 1) (layer "F.Cu") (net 3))
 (segment (start 129.46 39) (end 117.5113 50.9487) (width 1) (layer "F.Cu") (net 3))
 (segment (start 63 74.46) (end 57.6956 79.7644) (width 1) (layer "F.Cu") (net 3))
 (segment (start 117.5113 50.9487) (end 95.9141 50.9487) (width 1) (layer "F.Cu") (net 3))
 (segment (start 63.9559 72) (end 63 72.9559) (width 1) (layer "F.Cu") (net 3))
 (segment (start 79.0625 74) (end 72 74) (width 1) (layer "F.Cu") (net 3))
 (segment (start 70 72) (end 63.9559 72) (width 1) (layer "F.Cu") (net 3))
 (segment (start 57.6956 79.7644) (end 57.6956 92.0173) (width 1) (layer "F.Cu") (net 3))
 (segment (start 60.5 94.8217) (end 60.5 99) (width 1) (layer "F.Cu") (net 3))
 (segment (start 72 74) (end 70 72) (width 1) (layer "F.Cu") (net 3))
 (segment (start 63 74.46) (end 63 72.9559) (width 1) (layer "F.Cu") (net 3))
 (via (at 95.9141 50.9487) (size 0.8) (drill 0.4) (layers "F.Cu" "B.Cu") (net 3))
 (segment (start 74.8628 72) (end 70 72) (width 1) (layer "B.Cu") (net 3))
 (segment (start 95.9141 50.9487) (end 74.8628 72) (width 1) (layer "B.Cu") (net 3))
 (segment (start 63 81.0441) (end 61.75 82.2941) (width 1) (layer "B.Cu") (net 1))
 (segment (start 77.08 55.1041) (end 66.4731 65.711) (width 1) (layer "B.Cu") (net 1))
 (segment (start 66.4731 76.0669) (end 63 79.54) (width 1) (layer "B.Cu") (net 1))
 (segment (start 77.44 39) (end 77.44 51.0359) (width 1) (layer "B.Cu") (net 1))
 (segment (start 77.08 53.25) (end 77.08 55.1041) (width 1) (layer "B.Cu") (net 1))
 (segment (start 77.08 53.25) (end 77.08 51.3959) (width 1) (layer "B.Cu") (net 1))
 (segment (start 61.75 82.2941) (end 61.75 90) (width 1) (layer "B.Cu") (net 1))
 (segment (start 77.44 51.0359) (end 77.08 51.3959) (width 1) (layer "B.Cu") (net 1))
 (segment (start 66.4731 65.711) (end 66.4731 76.0669) (width 1) (layer "B.Cu") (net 1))
 (segment (start 63 79.54) (end 63 81.0441) (width 1) (layer "B.Cu") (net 1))
 (segment (start 63 77) (end 65.5 74.5) (width 1) (layer "F.Cu") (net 2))
 (segment (start 85.248 73.65) (end 82.8748 76.0232) (width 1) (layer "F.Cu") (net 2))
 (segment (start 74.9 39) (end 76.5265 37.3735) (width 1) (layer "F.Cu") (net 2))
 (segment (start 126.11 73.65) (end 85.248 73.65) (width 1) (layer "F.Cu") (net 2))
 (segment (start 65.5 74.5) (end 70 74.5) (width 1) (layer "F.Cu") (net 2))
 (segment (start 111.3735 37.3735) (end 113 39) (width 1) (layer "F.Cu") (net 2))
 (segment (start 76.5265 37.3735) (end 111.3735 37.3735) (width 1) (layer "F.Cu") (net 2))
 (segment (start 82.8748 76.0232) (end 71.5232 76.0232) (width 1) (layer "F.Cu") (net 2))
 (segment (start 71.5232 76.0232) (end 70 74.5) (width 1) (layer "F.Cu") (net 2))
 (segment (start 127.7228 75.2628) (end 127.7228 84.7372) (width 1) (layer "B.Cu") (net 2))
 (segment (start 60 74) (end 62.7606 76.7605) (width 1) (layer "B.Cu") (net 2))
 (segment (start 62.7606 76.7605) (end 63 77) (width 1) (layer "B.Cu") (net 2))
 (segment (start 127.7228 84.7372) (end 126.11 86.35) (width 1) (layer "B.Cu") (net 2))
 (segment (start 74.9 51.1) (end 60 66) (width 1) (layer "B.Cu") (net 2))
 (segment (start 59.25 80.2711) (end 62.7606 76.7605) (width 1) (layer "B.Cu") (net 2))
 (segment (start 126.11 60.95) (end 127.7142 62.5542) (width 1) (layer "B.Cu") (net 2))
 (segment (start 124.16 40.37) (end 122.5059 40.37) (width 1) (layer "B.Cu") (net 2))
 (segment (start 59 99) (end 59 90.25) (width 1) (layer "B.Cu") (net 2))
 (segment (start 127.7142 72.0458) (end 126.11 73.65) (width 1) (layer "B.Cu") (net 2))
 (segment (start 74.9 39) (end 74.9 51.1) (width 1) (layer "B.Cu") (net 2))
 (segment (start 126.11 73.65) (end 127.7228 75.2628) (width 1) (layer "B.Cu") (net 2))
 (segment (start 59 90.25) (end 59.25 90) (width 1) (layer "B.Cu") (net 2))
 (segment (start 127.7142 62.5542) (end 127.7142 72.0458) (width 1) (layer "B.Cu") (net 2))
 (segment (start 59.25 90) (end 59.25 80.2711) (width 1) (layer "B.Cu") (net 2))
 (segment (start 60 66) (end 60 74) (width 1) (layer "B.Cu") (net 2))
 (segment (start 122.5059 40.37) (end 121.1359 39) (width 1) (layer "B.Cu") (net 2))
 (segment (start 121.1359 39) (end 113 39) (width 1) (layer "B.Cu") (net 2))
 (segment (start 134.6693 37.7704) (end 135.8989 39) (width 0.254) (layer "F.Cu") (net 44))
 (segment (start 124.16 37.83) (end 124.2196 37.7704) (width 0.254) (layer "F.Cu") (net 44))
 (segment (start 124.2196 37.7704) (end 134.6693 37.7704) (width 0.254) (layer "F.Cu") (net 44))
 (segment (start 137.08 39) (end 135.8989 39) (width 0.254) (layer "F.Cu") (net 44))
 (segment (start 136.5952 64.7988) (end 141.6752 59.7188) (width 0.254) (layer "F.Cu") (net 40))
 (segment (start 80.9375 74.95) (end 91.0887 64.7988) (width 0.254) (layer "F.Cu") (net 40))
 (segment (start 146.6355 59.7188) (end 146.9212 59.4331) (width 0.254) (layer "F.Cu") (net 40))
 (segment (start 91.0887 64.7988) (end 136.5952 64.7988) (width 0.254) (layer "F.Cu") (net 40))
 (segment (start 146.9212 59.4331) (end 146.9212 57.3941) (width 0.254) (layer "F.Cu") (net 40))
 (segment (start 146.9212 57.3941) (end 145.3971 55.87) (width 0.254) (layer "F.Cu") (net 40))
 (segment (start 141.6752 59.7188) (end 146.6355 59.7188) (width 0.254) (layer "F.Cu") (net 40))
 (segment (start 145.3971 55.87) (end 143.89 55.87) (width 0.254) (layer "F.Cu") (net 40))
 (segment (start 80.9375 54.2113) (end 138.3546 54.2113) (width 1) (layer "F.Cu") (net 39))
 (segment (start 138.3546 54.2113) (end 142.2859 58.1426) (width 1) (layer "F.Cu") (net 39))
 (segment (start 143.89 58.41) (end 142.2859 58.41) (width 1) (layer "F.Cu") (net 39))
 (segment (start 79.98 39) (end 79.98 53.2538) (width 1) (layer "F.Cu") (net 39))
 (segment (start 80.9375 73.05) (end 80.9375 54.2113) (width 1) (layer "F.Cu") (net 39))
 (segment (start 142.2859 58.1426) (end 142.2859 58.41) (width 1) (layer "F.Cu") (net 39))
 (segment (start 79.98 53.2538) (end 80.9375 54.2113) (width 1) (layer "F.Cu") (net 39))
 (segment (start 66.92 53.25) (end 65.0659 53.25) (width 1) (layer "F.Cu") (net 45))
 (segment (start 60 55.5) (end 62.8159 55.5) (width 1) (layer "F.Cu") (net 45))
 (segment (start 62.8159 55.5) (end 65.0659 53.25) (width 1) (layer "F.Cu") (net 45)))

